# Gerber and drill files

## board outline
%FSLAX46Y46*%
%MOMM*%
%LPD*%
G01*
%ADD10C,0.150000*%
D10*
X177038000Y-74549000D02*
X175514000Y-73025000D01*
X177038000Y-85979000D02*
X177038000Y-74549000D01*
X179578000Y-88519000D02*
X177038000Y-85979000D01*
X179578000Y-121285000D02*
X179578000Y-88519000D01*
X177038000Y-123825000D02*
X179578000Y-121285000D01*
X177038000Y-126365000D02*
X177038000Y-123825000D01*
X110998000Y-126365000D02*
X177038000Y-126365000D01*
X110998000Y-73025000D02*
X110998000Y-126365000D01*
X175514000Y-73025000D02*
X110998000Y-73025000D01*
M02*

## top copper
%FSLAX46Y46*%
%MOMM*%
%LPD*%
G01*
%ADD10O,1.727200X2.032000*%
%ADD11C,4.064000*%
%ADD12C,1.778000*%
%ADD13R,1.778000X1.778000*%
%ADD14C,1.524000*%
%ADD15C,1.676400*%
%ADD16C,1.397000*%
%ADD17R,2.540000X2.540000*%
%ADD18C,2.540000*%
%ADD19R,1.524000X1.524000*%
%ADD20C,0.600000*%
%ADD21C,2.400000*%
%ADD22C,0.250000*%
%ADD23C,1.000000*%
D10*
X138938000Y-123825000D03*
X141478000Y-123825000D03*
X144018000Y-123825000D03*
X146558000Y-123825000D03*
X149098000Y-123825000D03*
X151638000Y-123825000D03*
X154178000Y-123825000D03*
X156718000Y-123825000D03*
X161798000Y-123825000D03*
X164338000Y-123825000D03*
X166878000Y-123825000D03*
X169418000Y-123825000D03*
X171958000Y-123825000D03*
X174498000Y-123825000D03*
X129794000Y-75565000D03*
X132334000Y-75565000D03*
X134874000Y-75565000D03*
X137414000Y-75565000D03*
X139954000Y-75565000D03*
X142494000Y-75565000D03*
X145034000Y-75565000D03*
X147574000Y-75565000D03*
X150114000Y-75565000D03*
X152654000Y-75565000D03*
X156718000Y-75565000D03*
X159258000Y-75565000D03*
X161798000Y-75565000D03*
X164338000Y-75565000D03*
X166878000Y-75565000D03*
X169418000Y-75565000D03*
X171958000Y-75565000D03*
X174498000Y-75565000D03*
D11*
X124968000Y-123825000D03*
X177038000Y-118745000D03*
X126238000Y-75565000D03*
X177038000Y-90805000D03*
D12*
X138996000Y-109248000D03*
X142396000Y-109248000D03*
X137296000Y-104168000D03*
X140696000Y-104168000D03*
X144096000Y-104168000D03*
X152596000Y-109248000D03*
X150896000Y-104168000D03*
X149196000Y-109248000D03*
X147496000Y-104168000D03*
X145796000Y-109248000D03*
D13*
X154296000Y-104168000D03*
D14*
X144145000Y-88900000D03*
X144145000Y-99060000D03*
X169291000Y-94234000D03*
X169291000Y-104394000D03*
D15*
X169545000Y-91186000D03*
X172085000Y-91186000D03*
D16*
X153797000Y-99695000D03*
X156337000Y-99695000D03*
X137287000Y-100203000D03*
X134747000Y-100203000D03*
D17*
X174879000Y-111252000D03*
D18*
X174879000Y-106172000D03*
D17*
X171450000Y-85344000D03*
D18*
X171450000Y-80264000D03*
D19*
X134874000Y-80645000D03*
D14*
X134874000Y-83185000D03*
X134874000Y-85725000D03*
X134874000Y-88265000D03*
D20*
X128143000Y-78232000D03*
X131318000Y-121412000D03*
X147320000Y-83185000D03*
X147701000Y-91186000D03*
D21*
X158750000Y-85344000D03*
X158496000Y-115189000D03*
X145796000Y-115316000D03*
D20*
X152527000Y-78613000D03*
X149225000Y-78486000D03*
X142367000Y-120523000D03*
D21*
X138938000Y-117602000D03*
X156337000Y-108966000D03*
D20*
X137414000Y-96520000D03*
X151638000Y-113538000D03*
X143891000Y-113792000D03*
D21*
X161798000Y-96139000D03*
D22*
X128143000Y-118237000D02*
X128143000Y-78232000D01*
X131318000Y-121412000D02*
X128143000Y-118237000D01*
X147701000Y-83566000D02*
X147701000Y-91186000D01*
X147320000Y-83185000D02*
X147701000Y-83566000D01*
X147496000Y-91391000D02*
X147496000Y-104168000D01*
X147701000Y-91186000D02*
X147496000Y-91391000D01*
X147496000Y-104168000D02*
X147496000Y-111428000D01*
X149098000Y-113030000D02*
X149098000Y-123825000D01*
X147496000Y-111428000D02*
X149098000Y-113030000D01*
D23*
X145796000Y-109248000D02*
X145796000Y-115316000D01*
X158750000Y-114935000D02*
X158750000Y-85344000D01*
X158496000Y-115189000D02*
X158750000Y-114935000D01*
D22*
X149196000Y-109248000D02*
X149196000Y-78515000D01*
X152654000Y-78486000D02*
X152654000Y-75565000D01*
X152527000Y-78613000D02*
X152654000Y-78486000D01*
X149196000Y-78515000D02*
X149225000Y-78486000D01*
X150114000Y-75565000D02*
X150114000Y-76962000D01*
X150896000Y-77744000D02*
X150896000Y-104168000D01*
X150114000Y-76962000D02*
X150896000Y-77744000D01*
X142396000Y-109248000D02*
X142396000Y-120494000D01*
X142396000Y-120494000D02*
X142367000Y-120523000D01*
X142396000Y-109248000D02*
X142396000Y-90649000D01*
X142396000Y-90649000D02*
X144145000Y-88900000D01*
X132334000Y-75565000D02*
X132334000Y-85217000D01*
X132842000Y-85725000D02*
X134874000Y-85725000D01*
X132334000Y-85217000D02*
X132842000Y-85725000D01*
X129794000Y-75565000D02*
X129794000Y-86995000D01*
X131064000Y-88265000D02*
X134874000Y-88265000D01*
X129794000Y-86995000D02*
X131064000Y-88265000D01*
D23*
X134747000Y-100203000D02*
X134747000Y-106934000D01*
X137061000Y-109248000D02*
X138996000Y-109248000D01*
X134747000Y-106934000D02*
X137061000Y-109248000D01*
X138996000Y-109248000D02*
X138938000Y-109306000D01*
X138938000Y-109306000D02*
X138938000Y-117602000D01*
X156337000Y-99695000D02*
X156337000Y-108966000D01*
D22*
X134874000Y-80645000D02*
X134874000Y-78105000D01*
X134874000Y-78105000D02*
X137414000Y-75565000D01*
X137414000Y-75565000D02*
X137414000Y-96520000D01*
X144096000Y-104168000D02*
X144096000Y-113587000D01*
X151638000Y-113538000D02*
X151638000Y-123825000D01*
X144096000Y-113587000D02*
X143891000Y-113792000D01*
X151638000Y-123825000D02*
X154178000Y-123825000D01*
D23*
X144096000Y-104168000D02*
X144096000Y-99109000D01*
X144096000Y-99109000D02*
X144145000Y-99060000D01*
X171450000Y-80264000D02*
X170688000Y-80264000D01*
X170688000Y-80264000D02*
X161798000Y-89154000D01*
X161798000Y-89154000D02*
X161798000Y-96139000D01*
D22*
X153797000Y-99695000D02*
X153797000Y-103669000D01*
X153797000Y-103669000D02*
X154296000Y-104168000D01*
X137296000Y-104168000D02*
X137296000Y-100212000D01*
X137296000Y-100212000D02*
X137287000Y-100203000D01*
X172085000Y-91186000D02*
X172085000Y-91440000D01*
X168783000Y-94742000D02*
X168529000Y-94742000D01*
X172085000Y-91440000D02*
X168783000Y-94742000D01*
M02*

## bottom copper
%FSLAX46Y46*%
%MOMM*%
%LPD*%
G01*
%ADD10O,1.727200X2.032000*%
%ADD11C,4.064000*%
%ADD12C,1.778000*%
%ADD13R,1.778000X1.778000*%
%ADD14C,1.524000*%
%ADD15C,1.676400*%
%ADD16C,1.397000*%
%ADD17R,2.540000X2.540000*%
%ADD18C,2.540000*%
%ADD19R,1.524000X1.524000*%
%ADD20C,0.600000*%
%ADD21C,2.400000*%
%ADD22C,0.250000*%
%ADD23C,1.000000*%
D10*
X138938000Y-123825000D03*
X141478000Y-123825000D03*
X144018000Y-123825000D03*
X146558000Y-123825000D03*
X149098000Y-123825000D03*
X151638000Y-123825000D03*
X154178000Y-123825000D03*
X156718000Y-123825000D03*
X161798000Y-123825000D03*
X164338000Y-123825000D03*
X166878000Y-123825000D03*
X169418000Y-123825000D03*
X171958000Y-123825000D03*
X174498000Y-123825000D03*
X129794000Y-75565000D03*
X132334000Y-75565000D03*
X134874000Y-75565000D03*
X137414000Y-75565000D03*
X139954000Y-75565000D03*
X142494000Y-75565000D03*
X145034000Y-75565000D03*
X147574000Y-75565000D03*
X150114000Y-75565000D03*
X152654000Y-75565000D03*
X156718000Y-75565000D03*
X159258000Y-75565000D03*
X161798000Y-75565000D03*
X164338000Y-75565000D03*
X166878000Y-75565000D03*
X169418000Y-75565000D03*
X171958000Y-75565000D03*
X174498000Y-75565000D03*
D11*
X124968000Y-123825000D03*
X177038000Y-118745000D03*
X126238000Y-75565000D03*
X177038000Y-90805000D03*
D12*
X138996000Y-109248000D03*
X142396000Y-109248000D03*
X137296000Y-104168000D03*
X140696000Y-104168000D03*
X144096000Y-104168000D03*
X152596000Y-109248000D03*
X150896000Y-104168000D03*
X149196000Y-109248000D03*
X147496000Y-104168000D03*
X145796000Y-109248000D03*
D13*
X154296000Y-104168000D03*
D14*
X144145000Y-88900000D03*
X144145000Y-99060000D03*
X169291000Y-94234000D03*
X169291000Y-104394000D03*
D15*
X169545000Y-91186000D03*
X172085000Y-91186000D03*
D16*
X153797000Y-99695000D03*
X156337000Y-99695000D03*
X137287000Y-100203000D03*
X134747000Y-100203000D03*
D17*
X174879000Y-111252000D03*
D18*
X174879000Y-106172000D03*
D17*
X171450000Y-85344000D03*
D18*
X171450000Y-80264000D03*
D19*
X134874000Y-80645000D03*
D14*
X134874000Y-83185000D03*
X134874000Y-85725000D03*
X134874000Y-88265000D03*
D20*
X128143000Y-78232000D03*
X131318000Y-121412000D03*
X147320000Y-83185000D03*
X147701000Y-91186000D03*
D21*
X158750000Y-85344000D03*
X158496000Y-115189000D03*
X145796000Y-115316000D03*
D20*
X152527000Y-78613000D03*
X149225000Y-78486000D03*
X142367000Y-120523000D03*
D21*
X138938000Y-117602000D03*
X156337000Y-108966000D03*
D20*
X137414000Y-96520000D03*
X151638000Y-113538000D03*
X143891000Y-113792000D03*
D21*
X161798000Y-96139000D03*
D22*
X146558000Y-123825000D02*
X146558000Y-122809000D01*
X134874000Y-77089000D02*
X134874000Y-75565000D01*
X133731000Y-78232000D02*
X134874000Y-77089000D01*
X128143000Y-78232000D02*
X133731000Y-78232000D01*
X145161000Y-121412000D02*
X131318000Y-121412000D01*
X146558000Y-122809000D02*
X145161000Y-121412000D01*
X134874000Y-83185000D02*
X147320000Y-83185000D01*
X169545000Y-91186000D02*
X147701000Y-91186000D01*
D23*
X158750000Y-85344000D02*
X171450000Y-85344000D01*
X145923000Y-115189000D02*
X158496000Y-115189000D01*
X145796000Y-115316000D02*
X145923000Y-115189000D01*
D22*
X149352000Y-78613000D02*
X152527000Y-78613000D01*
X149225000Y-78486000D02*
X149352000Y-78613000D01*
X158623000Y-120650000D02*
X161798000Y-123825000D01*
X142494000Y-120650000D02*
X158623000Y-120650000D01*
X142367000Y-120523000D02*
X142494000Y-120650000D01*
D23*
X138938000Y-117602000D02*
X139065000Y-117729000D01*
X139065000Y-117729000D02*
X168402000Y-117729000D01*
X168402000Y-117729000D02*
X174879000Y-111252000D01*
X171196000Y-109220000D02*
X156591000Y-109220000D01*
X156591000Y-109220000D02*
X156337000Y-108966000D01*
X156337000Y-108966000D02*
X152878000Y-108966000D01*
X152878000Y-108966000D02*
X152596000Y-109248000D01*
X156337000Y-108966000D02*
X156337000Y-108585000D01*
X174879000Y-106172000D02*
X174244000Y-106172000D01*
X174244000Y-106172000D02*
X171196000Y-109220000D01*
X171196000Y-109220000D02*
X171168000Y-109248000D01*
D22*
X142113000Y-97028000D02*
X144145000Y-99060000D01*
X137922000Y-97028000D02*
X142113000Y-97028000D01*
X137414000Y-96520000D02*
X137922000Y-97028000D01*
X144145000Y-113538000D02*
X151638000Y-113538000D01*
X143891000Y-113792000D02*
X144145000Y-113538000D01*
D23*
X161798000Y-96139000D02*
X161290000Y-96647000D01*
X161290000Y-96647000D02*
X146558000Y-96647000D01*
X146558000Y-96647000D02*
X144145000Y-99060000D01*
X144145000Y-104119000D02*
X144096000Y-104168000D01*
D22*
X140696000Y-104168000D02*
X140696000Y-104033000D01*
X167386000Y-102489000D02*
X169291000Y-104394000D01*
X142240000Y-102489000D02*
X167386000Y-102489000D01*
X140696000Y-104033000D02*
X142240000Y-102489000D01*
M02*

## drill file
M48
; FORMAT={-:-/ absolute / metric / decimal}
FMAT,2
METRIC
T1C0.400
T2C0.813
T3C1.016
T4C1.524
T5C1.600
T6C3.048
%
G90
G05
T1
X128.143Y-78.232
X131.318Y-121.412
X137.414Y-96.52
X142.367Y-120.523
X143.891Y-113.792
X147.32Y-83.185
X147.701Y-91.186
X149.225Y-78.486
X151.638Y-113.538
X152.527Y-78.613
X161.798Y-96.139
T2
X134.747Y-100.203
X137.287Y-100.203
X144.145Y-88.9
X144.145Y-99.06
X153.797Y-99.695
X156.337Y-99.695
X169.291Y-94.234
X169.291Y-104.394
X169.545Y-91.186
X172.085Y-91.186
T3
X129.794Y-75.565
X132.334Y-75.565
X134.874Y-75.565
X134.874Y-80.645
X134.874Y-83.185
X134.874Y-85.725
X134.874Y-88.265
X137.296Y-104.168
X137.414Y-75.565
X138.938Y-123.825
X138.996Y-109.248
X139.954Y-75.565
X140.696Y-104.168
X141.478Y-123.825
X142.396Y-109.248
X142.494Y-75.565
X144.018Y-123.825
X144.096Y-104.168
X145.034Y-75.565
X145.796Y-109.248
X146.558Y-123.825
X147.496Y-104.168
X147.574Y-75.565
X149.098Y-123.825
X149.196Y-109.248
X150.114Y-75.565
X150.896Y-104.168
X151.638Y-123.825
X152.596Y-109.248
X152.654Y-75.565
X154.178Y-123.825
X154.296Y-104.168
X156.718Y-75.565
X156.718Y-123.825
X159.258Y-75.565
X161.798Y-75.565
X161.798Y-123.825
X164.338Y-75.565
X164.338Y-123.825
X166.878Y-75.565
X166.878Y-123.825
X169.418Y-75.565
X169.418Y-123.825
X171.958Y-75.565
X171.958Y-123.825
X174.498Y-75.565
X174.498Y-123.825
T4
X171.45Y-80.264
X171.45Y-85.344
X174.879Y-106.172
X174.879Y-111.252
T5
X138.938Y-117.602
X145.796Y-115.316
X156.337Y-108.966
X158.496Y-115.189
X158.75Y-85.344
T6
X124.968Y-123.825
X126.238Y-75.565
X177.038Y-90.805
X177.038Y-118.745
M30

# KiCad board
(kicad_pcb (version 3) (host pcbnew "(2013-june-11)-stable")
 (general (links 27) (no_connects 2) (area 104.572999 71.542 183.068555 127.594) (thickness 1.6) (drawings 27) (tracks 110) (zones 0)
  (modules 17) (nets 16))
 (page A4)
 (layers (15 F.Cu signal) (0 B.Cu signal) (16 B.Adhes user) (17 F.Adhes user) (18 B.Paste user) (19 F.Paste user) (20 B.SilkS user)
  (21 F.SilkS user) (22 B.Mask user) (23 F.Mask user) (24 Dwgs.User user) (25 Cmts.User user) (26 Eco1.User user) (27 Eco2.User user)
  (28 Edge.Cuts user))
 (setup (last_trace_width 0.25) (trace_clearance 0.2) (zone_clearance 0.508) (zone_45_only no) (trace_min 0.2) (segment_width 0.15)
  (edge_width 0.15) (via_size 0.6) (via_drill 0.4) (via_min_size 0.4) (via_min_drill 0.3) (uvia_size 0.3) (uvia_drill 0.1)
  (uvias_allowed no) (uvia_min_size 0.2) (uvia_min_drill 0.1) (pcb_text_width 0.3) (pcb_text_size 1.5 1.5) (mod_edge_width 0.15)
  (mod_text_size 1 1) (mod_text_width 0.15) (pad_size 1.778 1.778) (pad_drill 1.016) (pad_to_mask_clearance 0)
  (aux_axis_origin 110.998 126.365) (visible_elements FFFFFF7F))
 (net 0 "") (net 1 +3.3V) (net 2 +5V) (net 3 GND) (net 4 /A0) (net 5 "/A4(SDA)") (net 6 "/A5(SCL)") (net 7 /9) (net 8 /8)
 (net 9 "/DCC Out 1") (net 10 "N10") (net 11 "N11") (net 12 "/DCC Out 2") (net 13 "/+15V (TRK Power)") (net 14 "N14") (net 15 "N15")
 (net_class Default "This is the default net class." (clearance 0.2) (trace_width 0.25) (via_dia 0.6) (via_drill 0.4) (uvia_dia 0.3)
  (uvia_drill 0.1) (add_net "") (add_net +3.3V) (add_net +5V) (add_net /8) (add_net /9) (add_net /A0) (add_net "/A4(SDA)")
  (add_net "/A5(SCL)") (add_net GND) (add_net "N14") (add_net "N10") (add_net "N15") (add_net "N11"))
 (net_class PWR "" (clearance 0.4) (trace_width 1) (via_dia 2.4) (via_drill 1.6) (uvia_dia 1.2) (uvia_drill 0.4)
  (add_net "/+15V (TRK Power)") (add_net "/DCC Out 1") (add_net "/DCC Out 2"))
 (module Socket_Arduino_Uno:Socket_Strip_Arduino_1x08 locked (layer F.Cu) (at 138.938 123.825)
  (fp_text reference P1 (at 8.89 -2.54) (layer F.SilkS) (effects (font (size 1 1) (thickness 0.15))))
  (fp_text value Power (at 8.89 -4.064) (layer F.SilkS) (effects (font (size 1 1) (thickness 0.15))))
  (pad 1 thru_hole oval (at 0 0) (size 1.7272 2.032) (drill 1.016) (layers *.Cu *.Mask F.SilkS))
  (pad 2 thru_hole oval (at 2.54 0) (size 1.7272 2.032) (drill 1.016) (layers *.Cu *.Mask F.SilkS))
  (pad 3 thru_hole oval (at 5.08 0) (size 1.7272 2.032) (drill 1.016) (layers *.Cu *.Mask F.SilkS))
  (pad 4 thru_hole oval (at 7.62 0) (size 1.7272 2.032) (drill 1.016) (layers *.Cu *.Mask F.SilkS) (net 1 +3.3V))
  (pad 5 thru_hole oval (at 10.16 0) (size 1.7272 2.032) (drill 1.016) (layers *.Cu *.Mask F.SilkS) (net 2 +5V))
  (pad 6 thru_hole oval (at 12.7 0) (size 1.7272 2.032) (drill 1.016) (layers *.Cu *.Mask F.SilkS) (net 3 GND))
  (pad 7 thru_hole oval (at 15.24 0) (size 1.7272 2.032) (drill 1.016) (layers *.Cu *.Mask F.SilkS) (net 3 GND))
  (pad 8 thru_hole oval (at 17.78 0) (size 1.7272 2.032) (drill 1.016) (layers *.Cu *.Mask F.SilkS)))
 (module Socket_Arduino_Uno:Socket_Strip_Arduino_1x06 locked (layer F.Cu) (at 161.798 123.825)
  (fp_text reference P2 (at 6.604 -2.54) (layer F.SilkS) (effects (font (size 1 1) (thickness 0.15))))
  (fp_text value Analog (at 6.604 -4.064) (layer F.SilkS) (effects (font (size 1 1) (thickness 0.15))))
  (pad 1 thru_hole oval (at 0 0) (size 1.7272 2.032) (drill 1.016) (layers *.Cu *.Mask F.SilkS) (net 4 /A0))
  (pad 2 thru_hole oval (at 2.54 0) (size 1.7272 2.032) (drill 1.016) (layers *.Cu *.Mask F.SilkS))
  (pad 3 thru_hole oval (at 5.08 0) (size 1.7272 2.032) (drill 1.016) (layers *.Cu *.Mask F.SilkS))
  (pad 4 thru_hole oval (at 7.62 0) (size 1.7272 2.032) (drill 1.016) (layers *.Cu *.Mask F.SilkS))
  (pad 5 thru_hole oval (at 10.16 0) (size 1.7272 2.032) (drill 1.016) (layers *.Cu *.Mask F.SilkS) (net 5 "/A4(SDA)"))
  (pad 6 thru_hole oval (at 12.7 0) (size 1.7272 2.032) (drill 1.016) (layers *.Cu *.Mask F.SilkS) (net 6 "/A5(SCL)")))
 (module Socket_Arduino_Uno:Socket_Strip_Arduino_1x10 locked (layer F.Cu) (at 129.794 75.565)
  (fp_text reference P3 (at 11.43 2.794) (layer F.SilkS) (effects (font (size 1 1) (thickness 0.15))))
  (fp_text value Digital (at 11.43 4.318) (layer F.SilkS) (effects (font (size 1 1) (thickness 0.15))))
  (pad 1 thru_hole oval (at 0 0) (size 1.7272 2.032) (drill 1.016) (layers *.Cu *.Mask F.SilkS) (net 6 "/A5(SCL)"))
  (pad 2 thru_hole oval (at 2.54 0) (size 1.7272 2.032) (drill 1.016) (layers *.Cu *.Mask F.SilkS) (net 5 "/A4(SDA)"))
  (pad 3 thru_hole oval (at 5.08 0) (size 1.7272 2.032) (drill 1.016) (layers *.Cu *.Mask F.SilkS) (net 1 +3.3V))
  (pad 4 thru_hole oval (at 7.62 0) (size 1.7272 2.032) (drill 1.016) (layers *.Cu *.Mask F.SilkS) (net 3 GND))
  (pad 5 thru_hole oval (at 10.16 0) (size 1.7272 2.032) (drill 1.016) (layers *.Cu *.Mask F.SilkS))
  (pad 6 thru_hole oval (at 12.7 0) (size 1.7272 2.032) (drill 1.016) (layers *.Cu *.Mask F.SilkS))
  (pad 7 thru_hole oval (at 15.24 0) (size 1.7272 2.032) (drill 1.016) (layers *.Cu *.Mask F.SilkS))
  (pad 8 thru_hole oval (at 17.78 0) (size 1.7272 2.032) (drill 1.016) (layers *.Cu *.Mask F.SilkS))
  (pad 9 thru_hole oval (at 20.32 0) (size 1.7272 2.032) (drill 1.016) (layers *.Cu *.Mask F.SilkS) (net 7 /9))
  (pad 10 thru_hole oval (at 22.86 0) (size 1.7272 2.032) (drill 1.016) (layers *.Cu *.Mask F.SilkS) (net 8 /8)))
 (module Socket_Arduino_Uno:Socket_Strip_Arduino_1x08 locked (layer F.Cu) (at 156.718 75.565)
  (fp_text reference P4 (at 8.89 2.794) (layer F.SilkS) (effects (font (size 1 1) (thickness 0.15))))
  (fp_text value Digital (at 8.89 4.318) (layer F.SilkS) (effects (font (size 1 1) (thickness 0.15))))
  (pad 1 thru_hole oval (at 0 0) (size 1.7272 2.032) (drill 1.016) (layers *.Cu *.Mask F.SilkS))
  (pad 2 thru_hole oval (at 2.54 0) (size 1.7272 2.032) (drill 1.016) (layers *.Cu *.Mask F.SilkS))
  (pad 3 thru_hole oval (at 5.08 0) (size 1.7272 2.032) (drill 1.016) (layers *.Cu *.Mask F.SilkS))
  (pad 4 thru_hole oval (at 7.62 0) (size 1.7272 2.032) (drill 1.016) (layers *.Cu *.Mask F.SilkS))
  (pad 5 thru_hole oval (at 10.16 0) (size 1.7272 2.032) (drill 1.016) (layers *.Cu *.Mask F.SilkS))
  (pad 6 thru_hole oval (at 12.7 0) (size 1.7272 2.032) (drill 1.016) (layers *.Cu *.Mask F.SilkS))
  (pad 7 thru_hole oval (at 15.24 0) (size 1.7272 2.032) (drill 1.016) (layers *.Cu *.Mask F.SilkS))
  (pad 8 thru_hole oval (at 17.78 0) (size 1.7272 2.032) (drill 1.016) (layers *.Cu *.Mask F.SilkS)))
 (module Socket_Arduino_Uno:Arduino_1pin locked (layer F.Cu) (at 124.968 123.825)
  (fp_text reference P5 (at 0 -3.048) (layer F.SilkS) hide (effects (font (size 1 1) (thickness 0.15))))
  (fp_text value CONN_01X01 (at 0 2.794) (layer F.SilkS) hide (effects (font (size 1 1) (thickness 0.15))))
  (pad 1 thru_hole circle (at 0 0) (size 4.064 4.064) (drill 3.048) (layers *.Cu *.Mask F.SilkS)))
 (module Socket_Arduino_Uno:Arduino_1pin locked (layer F.Cu) (at 177.038 118.745)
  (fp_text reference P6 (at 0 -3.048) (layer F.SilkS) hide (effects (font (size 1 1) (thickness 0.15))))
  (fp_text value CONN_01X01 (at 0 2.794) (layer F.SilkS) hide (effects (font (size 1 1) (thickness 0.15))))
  (pad 1 thru_hole circle (at 0 0) (size 4.064 4.064) (drill 3.048) (layers *.Cu *.Mask F.SilkS)))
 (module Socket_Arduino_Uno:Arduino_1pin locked (layer F.Cu) (at 126.238 75.565)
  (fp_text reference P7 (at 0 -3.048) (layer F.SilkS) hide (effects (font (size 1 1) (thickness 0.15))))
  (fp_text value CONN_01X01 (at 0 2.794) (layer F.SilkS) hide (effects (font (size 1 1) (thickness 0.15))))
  (pad 1 thru_hole circle (at 0 0) (size 4.064 4.064) (drill 3.048) (layers *.Cu *.Mask F.SilkS)))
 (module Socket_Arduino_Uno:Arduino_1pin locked (layer F.Cu) (at 177.038 90.805)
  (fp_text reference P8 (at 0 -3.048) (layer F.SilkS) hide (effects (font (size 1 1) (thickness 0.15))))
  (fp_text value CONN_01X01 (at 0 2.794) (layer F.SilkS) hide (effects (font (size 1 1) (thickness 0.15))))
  (pad 1 thru_hole circle (at 0 0) (size 4.064 4.064) (drill 3.048) (layers *.Cu *.Mask F.SilkS)))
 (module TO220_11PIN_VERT (layer F.Cu) (at 145.796 110.998 270)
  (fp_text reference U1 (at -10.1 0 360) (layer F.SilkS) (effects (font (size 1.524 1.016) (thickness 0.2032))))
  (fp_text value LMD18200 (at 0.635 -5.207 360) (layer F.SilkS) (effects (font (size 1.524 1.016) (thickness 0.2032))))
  (pad 10 thru_hole circle (at -1.75 6.8 270) (size 1.778 1.778) (drill 1.016) (layers *.Cu *.Mask F.SilkS) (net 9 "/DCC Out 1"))
  (pad 8 thru_hole circle (at -1.75 3.4 270) (size 1.778 1.778) (drill 1.016) (layers *.Cu *.Mask F.SilkS) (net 4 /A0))
  (pad 11 thru_hole circle (at -6.83 8.5 270) (size 1.778 1.778) (drill 1.016) (layers *.Cu *.Mask F.SilkS) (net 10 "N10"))
  (pad 9 thru_hole circle (at -6.83 5.1 270) (size 1.778 1.778) (drill 1.016) (layers *.Cu *.Mask F.SilkS) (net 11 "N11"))
  (pad 7 thru_hole circle (at -6.83 1.7 270) (size 1.778 1.778) (drill 1.016) (layers *.Cu *.Mask F.SilkS) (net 3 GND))
  (pad 2 thru_hole circle (at -1.75 -6.8 270) (size 1.778 1.778) (drill 1.016) (layers *.Cu *.Mask F.SilkS) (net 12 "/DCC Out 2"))
  (pad 3 thru_hole circle (at -6.83 -5.1 270) (size 1.778 1.778) (drill 1.016) (layers *.Cu *.Mask F.SilkS) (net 7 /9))
  (pad 4 thru_hole circle (at -1.75 -3.4 270) (size 1.778 1.778) (drill 1.016) (layers *.Cu *.Mask F.SilkS) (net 8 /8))
  (pad 5 thru_hole circle (at -6.83 -1.7 270) (size 1.778 1.778) (drill 1.016) (layers *.Cu *.Mask F.SilkS) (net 2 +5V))
  (pad 6 thru_hole circle (at -1.75 0 270) (size 1.778 1.778) (drill 1.016) (layers *.Cu *.Mask F.SilkS) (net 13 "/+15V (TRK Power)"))
  (pad 1 thru_hole rect (at -6.83 -8.5 270) (size 1.778 1.778) (drill 1.016) (layers *.Cu *.Mask F.SilkS) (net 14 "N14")))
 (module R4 (layer F.Cu) (at 144.145 93.98 270) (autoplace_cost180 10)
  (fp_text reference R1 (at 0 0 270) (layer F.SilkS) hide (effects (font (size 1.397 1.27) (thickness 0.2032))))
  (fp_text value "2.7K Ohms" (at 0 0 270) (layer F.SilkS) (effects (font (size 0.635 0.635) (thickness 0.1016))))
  (pad 1 thru_hole circle (at -5.08 0 270) (size 1.524 1.524) (drill 0.8128) (layers *.Cu *.Mask F.SilkS) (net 4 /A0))
  (pad 2 thru_hole circle (at 5.08 0 270) (size 1.524 1.524) (drill 0.8128) (layers *.Cu *.Mask F.SilkS) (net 3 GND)))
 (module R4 (layer F.Cu) (at 169.291 99.314 270) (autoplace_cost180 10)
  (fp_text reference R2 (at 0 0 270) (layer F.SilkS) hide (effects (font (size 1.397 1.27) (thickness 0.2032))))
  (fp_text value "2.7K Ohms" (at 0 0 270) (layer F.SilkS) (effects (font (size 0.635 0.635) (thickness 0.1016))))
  (pad 1 thru_hole circle (at -5.08 0 270) (size 1.524 1.524) (drill 0.8128) (layers *.Cu *.Mask F.SilkS) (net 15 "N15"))
  (pad 2 thru_hole circle (at 5.08 0 270) (size 1.524 1.524) (drill 0.8128) (layers *.Cu *.Mask F.SilkS) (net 11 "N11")))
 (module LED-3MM (layer F.Cu) (at 170.815 91.186)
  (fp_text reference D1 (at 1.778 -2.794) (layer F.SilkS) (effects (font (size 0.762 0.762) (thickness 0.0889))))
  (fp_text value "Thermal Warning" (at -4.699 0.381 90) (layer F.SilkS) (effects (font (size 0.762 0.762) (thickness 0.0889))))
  (pad 1 thru_hole circle (at -1.27 0) (size 1.6764 1.6764) (drill 0.8128) (layers *.Cu *.Mask F.SilkS) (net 2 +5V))
  (pad 2 thru_hole circle (at 1.27 0) (size 1.6764 1.6764) (drill 0.8128) (layers *.Cu *.Mask F.SilkS) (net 15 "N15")))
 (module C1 (layer F.Cu) (at 155.067 99.695)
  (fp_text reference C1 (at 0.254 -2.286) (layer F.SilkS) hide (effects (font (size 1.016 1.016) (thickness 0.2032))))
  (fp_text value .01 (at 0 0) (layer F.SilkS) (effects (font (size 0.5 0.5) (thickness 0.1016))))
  (pad 1 thru_hole circle (at -1.27 0) (size 1.397 1.397) (drill 0.8128) (layers *.Cu *.Mask F.SilkS) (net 14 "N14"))
  (pad 2 thru_hole circle (at 1.27 0) (size 1.397 1.397) (drill 0.8128) (layers *.Cu *.Mask F.SilkS) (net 12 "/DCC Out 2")))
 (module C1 (layer F.Cu) (at 136.017 100.203 180)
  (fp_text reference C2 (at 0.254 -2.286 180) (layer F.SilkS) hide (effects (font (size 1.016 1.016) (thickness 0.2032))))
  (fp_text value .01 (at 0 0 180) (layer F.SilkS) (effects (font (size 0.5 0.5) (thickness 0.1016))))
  (pad 1 thru_hole circle (at -1.27 0 180) (size 1.397 1.397) (drill 0.8128) (layers *.Cu *.Mask F.SilkS) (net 10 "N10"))
  (pad 2 thru_hole circle (at 1.27 0 180) (size 1.397 1.397) (drill 0.8128) (layers *.Cu *.Mask F.SilkS) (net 9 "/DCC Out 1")))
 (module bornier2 (layer F.Cu) (at 174.879 108.712 90)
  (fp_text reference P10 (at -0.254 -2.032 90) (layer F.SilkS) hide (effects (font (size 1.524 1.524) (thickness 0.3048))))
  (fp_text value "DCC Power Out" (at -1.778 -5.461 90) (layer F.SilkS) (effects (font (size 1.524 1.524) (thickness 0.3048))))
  (pad 1 thru_hole rect (at -2.54 0 90) (size 2.54 2.54) (drill 1.524) (layers *.Cu *.Mask F.SilkS) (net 9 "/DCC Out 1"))
  (pad 2 thru_hole circle (at 2.54 0 90) (size 2.54 2.54) (drill 1.524) (layers *.Cu *.Mask F.SilkS) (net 12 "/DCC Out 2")))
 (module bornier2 (layer F.Cu) (at 171.45 82.804 90)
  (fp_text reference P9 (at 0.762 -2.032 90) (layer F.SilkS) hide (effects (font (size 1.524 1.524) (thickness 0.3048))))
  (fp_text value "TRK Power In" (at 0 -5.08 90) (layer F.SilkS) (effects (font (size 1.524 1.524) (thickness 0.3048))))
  (pad 1 thru_hole rect (at -2.54 0 90) (size 2.54 2.54) (drill 1.524) (layers *.Cu *.Mask F.SilkS) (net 13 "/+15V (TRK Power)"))
  (pad 2 thru_hole circle (at 2.54 0 90) (size 2.54 2.54) (drill 1.524) (layers *.Cu *.Mask F.SilkS) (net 3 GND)))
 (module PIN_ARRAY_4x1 (layer F.Cu) (at 134.874 84.455 270)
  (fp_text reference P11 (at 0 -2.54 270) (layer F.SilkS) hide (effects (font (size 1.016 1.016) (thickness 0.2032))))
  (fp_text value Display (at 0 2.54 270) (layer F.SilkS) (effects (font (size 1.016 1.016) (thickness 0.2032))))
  (pad 1 thru_hole rect (at -3.81 0 270) (size 1.524 1.524) (drill 1.016) (layers *.Cu *.Mask F.SilkS) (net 3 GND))
  (pad 2 thru_hole circle (at -1.27 0 270) (size 1.524 1.524) (drill 1.016) (layers *.Cu *.Mask F.SilkS) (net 2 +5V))
  (pad 3 thru_hole circle (at 1.27 0 270) (size 1.524 1.524) (drill 1.016) (layers *.Cu *.Mask F.SilkS) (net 5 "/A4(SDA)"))
  (pad 4 thru_hole circle (at 3.81 0 270) (size 1.524 1.524) (drill 1.016) (layers *.Cu *.Mask F.SilkS) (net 6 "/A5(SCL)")))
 (gr_line (start 177.038 74.549) (end 175.514 73.025) (angle 90) (layer Edge.Cuts) (width 0.15))
 (gr_line (start 177.038 85.979) (end 177.038 74.549) (angle 90) (layer Edge.Cuts) (width 0.15))
 (gr_line (start 179.578 88.519) (end 177.038 85.979) (angle 90) (layer Edge.Cuts) (width 0.15))
 (gr_line (start 179.578 121.285) (end 179.578 88.519) (angle 90) (layer Edge.Cuts) (width 0.15))
 (gr_line (start 177.038 123.825) (end 179.578 121.285) (angle 90) (layer Edge.Cuts) (width 0.15))
 (gr_line (start 177.038 126.365) (end 177.038 123.825) (angle 90) (layer Edge.Cuts) (width 0.15))
 (gr_line (start 110.998 126.365) (end 177.038 126.365) (angle 90) (layer Edge.Cuts) (width 0.15))
 (gr_line (start 110.998 73.025) (end 110.998 126.365) (angle 90) (layer Edge.Cuts) (width 0.15))
 (gr_line (start 175.514 73.025) (end 110.998 73.025) (angle 90) (layer Edge.Cuts) (width 0.15))
 (segment (start 146.558 123.825) (end 146.558 122.809) (width 0.25) (layer B.Cu) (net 1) (status C00000))
 (segment (start 134.874 77.089) (end 134.874 75.565) (width 0.25) (layer B.Cu) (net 1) (status 800000))
 (segment (start 133.731 78.232) (end 134.874 77.089) (width 0.25) (layer B.Cu) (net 1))
 (segment (start 128.143 78.232) (end 133.731 78.232) (width 0.25) (layer B.Cu) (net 1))
 (via (at 128.143 78.232) (size 0.6) (layers F.Cu B.Cu) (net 1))
 (segment (start 128.143 118.237) (end 128.143 78.232) (width 0.25) (layer F.Cu) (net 1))
 (segment (start 131.318 121.412) (end 128.143 118.237) (width 0.25) (layer F.Cu) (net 1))
 (via (at 131.318 121.412) (size 0.6) (layers F.Cu B.Cu) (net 1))
 (segment (start 145.161 121.412) (end 131.318 121.412) (width 0.25) (layer B.Cu) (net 1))
 (segment (start 146.558 122.809) (end 145.161 121.412) (width 0.25) (layer B.Cu) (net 1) (status 400000))
 (segment (start 134.874 83.185) (end 147.32 83.185) (width 0.25) (layer B.Cu) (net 2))
 (segment (start 147.701 83.566) (end 147.701 91.186) (width 0.25) (layer F.Cu) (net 2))
 (segment (start 147.32 83.185) (end 147.701 83.566) (width 0.25) (layer F.Cu) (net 2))
 (via (at 147.32 83.185) (size 0.6) (layers F.Cu B.Cu) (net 2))
 (segment (start 169.545 91.186) (end 147.701 91.186) (width 0.25) (layer B.Cu) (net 2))
 (segment (start 147.496 91.391) (end 147.496 104.168) (width 0.25) (layer F.Cu) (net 2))
 (segment (start 147.701 91.186) (end 147.496 91.391) (width 0.25) (layer F.Cu) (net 2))
 (via (at 147.701 91.186) (size 0.6) (layers F.Cu B.Cu) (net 2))
 (segment (start 147.496 104.168) (end 147.496 111.428) (width 0.25) (layer F.Cu) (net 2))
 (segment (start 149.098 113.03) (end 149.098 123.825) (width 0.25) (layer F.Cu) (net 2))
 (segment (start 147.496 111.428) (end 149.098 113.03) (width 0.25) (layer F.Cu) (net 2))
 (segment (start 145.796 109.248) (end 145.796 115.316) (width 1) (layer F.Cu) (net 13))
 (segment (start 158.75 85.344) (end 171.45 85.344) (width 1) (layer B.Cu) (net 13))
 (via (at 158.75 85.344) (size 2.4) (layers F.Cu B.Cu) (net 13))
 (segment (start 158.75 114.935) (end 158.75 85.344) (width 1) (layer F.Cu) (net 13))
 (segment (start 158.496 115.189) (end 158.75 114.935) (width 1) (layer F.Cu) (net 13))
 (via (at 158.496 115.189) (size 2.4) (layers F.Cu B.Cu) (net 13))
 (segment (start 145.923 115.189) (end 158.496 115.189) (width 1) (layer B.Cu) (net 13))
 (segment (start 145.796 115.316) (end 145.923 115.189) (width 1) (layer B.Cu) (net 13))
 (via (at 145.796 115.316) (size 2.4) (layers F.Cu B.Cu) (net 13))
 (segment (start 149.196 109.248) (end 149.196 78.515) (width 0.25) (layer F.Cu) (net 8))
 (segment (start 152.654 78.486) (end 152.654 75.565) (width 0.25) (layer F.Cu) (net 8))
 (segment (start 152.527 78.613) (end 152.654 78.486) (width 0.25) (layer F.Cu) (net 8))
 (via (at 152.527 78.613) (size 0.6) (layers F.Cu B.Cu) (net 8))
 (segment (start 149.352 78.613) (end 152.527 78.613) (width 0.25) (layer B.Cu) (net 8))
 (segment (start 149.225 78.486) (end 149.352 78.613) (width 0.25) (layer B.Cu) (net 8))
 (via (at 149.225 78.486) (size 0.6) (layers F.Cu B.Cu) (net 8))
 (segment (start 149.196 78.515) (end 149.225 78.486) (width 0.25) (layer F.Cu) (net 8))
 (segment (start 150.114 75.565) (end 150.114 76.962) (width 0.25) (layer F.Cu) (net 7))
 (segment (start 150.896 77.744) (end 150.896 104.168) (width 0.25) (layer F.Cu) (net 7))
 (segment (start 150.114 76.962) (end 150.896 77.744) (width 0.25) (layer F.Cu) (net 7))
 (segment (start 142.396 109.248) (end 142.396 120.494) (width 0.25) (layer F.Cu) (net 4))
 (segment (start 158.623 120.65) (end 161.798 123.825) (width 0.25) (layer B.Cu) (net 4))
 (segment (start 142.494 120.65) (end 158.623 120.65) (width 0.25) (layer B.Cu) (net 4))
 (segment (start 142.367 120.523) (end 142.494 120.65) (width 0.25) (layer B.Cu) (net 4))
 (via (at 142.367 120.523) (size 0.6) (layers F.Cu B.Cu) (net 4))
 (segment (start 142.396 120.494) (end 142.367 120.523) (width 0.25) (layer F.Cu) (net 4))
 (segment (start 142.396 109.248) (end 142.396 90.649) (width 0.25) (layer F.Cu) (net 4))
 (segment (start 142.396 90.649) (end 144.145 88.9) (width 0.25) (layer F.Cu) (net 4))
 (segment (start 132.334 75.565) (end 132.334 85.217) (width 0.25) (layer F.Cu) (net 5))
 (segment (start 132.842 85.725) (end 134.874 85.725) (width 0.25) (layer F.Cu) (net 5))
 (segment (start 132.334 85.217) (end 132.842 85.725) (width 0.25) (layer F.Cu) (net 5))
 (segment (start 129.794 75.565) (end 129.794 86.995) (width 0.25) (layer F.Cu) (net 6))
 (segment (start 131.064 88.265) (end 134.874 88.265) (width 0.25) (layer F.Cu) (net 6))
 (segment (start 129.794 86.995) (end 131.064 88.265) (width 0.25) (layer F.Cu) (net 6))
 (segment (start 134.747 100.203) (end 134.747 106.934) (width 1) (layer F.Cu) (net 9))
 (segment (start 137.061 109.248) (end 138.996 109.248) (width 1) (layer F.Cu) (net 9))
 (segment (start 134.747 106.934) (end 137.061 109.248) (width 1) (layer F.Cu) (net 9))
 (segment (start 138.996 109.248) (end 138.938 109.306) (width 1) (layer F.Cu) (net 9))
 (segment (start 138.938 109.306) (end 138.938 117.602) (width 1) (layer F.Cu) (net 9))
 (via (at 138.938 117.602) (size 2.4) (layers F.Cu B.Cu) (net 9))
 (segment (start 138.938 117.602) (end 139.065 117.729) (width 1) (layer B.Cu) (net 9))
 (segment (start 139.065 117.729) (end 168.402 117.729) (width 1) (layer B.Cu) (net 9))
 (segment (start 168.402 117.729) (end 174.879 111.252) (width 1) (layer B.Cu) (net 9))
 (segment (start 171.196 109.22) (end 156.591 109.22) (width 1) (layer B.Cu) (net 12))
 (segment (start 156.591 109.22) (end 156.337 108.966) (width 1) (layer B.Cu) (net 12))
 (segment (start 156.337 108.966) (end 152.878 108.966) (width 1) (layer B.Cu) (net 12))
 (segment (start 152.878 108.966) (end 152.596 109.248) (width 1) (layer B.Cu) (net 12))
 (segment (start 156.337 99.695) (end 156.337 108.966) (width 1) (layer F.Cu) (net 12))
 (via (at 156.337 108.966) (size 2.4) (layers F.Cu B.Cu) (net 12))
 (segment (start 156.337 108.966) (end 156.337 108.585) (width 1) (layer B.Cu) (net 12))
 (segment (start 174.879 106.172) (end 174.244 106.172) (width 1) (layer B.Cu) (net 12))
 (segment (start 174.244 106.172) (end 171.196 109.22) (width 1) (layer B.Cu) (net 12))
 (segment (start 171.196 109.22) (end 171.168 109.248) (width 1) (layer B.Cu) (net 12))
 (segment (start 134.874 80.645) (end 134.874 78.105) (width 0.25) (layer F.Cu) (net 3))
 (segment (start 134.874 78.105) (end 137.414 75.565) (width 0.25) (layer F.Cu) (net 3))
 (segment (start 137.414 75.565) (end 137.414 96.52) (width 0.25) (layer F.Cu) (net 3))
 (segment (start 142.113 97.028) (end 144.145 99.06) (width 0.25) (layer B.Cu) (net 3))
 (segment (start 137.922 97.028) (end 142.113 97.028) (width 0.25) (layer B.Cu) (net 3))
 (segment (start 137.414 96.52) (end 137.922 97.028) (width 0.25) (layer B.Cu) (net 3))
 (via (at 137.414 96.52) (size 0.6) (layers F.Cu B.Cu) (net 3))
 (segment (start 144.096 104.168) (end 144.096 113.587) (width 0.25) (layer F.Cu) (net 3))
 (segment (start 151.638 113.538) (end 151.638 123.825) (width 0.25) (layer F.Cu) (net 3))
 (via (at 151.638 113.538) (size 0.6) (layers F.Cu B.Cu) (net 3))
 (segment (start 144.145 113.538) (end 151.638 113.538) (width 0.25) (layer B.Cu) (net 3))
 (segment (start 143.891 113.792) (end 144.145 113.538) (width 0.25) (layer B.Cu) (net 3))
 (via (at 143.891 113.792) (size 0.6) (layers F.Cu B.Cu) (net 3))
 (segment (start 144.096 113.587) (end 143.891 113.792) (width 0.25) (layer F.Cu) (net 3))
 (segment (start 151.638 123.825) (end 154.178 123.825) (width 0.25) (layer F.Cu) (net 3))
 (segment (start 144.096 104.168) (end 144.096 99.109) (width 1) (layer F.Cu) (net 3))
 (segment (start 144.096 99.109) (end 144.145 99.06) (width 1) (layer F.Cu) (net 3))
 (segment (start 171.45 80.264) (end 170.688 80.264) (width 1) (layer F.Cu) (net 3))
 (segment (start 170.688 80.264) (end 161.798 89.154) (width 1) (layer F.Cu) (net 3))
 (segment (start 161.798 89.154) (end 161.798 96.139) (width 1) (layer F.Cu) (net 3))
 (via (at 161.798 96.139) (size 2.4) (layers F.Cu B.Cu) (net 3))
 (segment (start 161.798 96.139) (end 161.29 96.647) (width 1) (layer B.Cu) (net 3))
 (segment (start 161.29 96.647) (end 146.558 96.647) (width 1) (layer B.Cu) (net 3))
 (segment (start 146.558 96.647) (end 144.145 99.06) (width 1) (layer B.Cu) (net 3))
 (segment (start 144.145 104.119) (end 144.096 104.168) (width 1) (layer B.Cu) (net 3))
 (segment (start 153.797 99.695) (end 153.797 103.669) (width 0.25) (layer F.Cu) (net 14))
 (segment (start 153.797 103.669) (end 154.296 104.168) (width 0.25) (layer F.Cu) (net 14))
 (segment (start 137.296 104.168) (end 137.296 100.212) (width 0.25) (layer F.Cu) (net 10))
 (segment (start 137.296 100.212) (end 137.287 100.203) (width 0.25) (layer F.Cu) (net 10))
 (segment (start 172.085 91.186) (end 172.085 91.44) (width 0.25) (layer F.Cu) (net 15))
 (segment (start 168.783 94.742) (end 168.529 94.742) (width 0.25) (layer F.Cu) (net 15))
 (segment (start 172.085 91.44) (end 168.783 94.742) (width 0.25) (layer F.Cu) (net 15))
 (segment (start 140.696 104.168) (end 140.696 104.033) (width 0.25) (layer B.Cu) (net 11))
 (segment (start 167.386 102.489) (end 169.291 104.394) (width 0.25) (layer B.Cu) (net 11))
 (segment (start 142.24 102.489) (end 167.386 102.489) (width 0.25) (layer B.Cu) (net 11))
 (segment (start 140.696 104.033) (end 142.24 102.489) (width 0.25) (layer B.Cu) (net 11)))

